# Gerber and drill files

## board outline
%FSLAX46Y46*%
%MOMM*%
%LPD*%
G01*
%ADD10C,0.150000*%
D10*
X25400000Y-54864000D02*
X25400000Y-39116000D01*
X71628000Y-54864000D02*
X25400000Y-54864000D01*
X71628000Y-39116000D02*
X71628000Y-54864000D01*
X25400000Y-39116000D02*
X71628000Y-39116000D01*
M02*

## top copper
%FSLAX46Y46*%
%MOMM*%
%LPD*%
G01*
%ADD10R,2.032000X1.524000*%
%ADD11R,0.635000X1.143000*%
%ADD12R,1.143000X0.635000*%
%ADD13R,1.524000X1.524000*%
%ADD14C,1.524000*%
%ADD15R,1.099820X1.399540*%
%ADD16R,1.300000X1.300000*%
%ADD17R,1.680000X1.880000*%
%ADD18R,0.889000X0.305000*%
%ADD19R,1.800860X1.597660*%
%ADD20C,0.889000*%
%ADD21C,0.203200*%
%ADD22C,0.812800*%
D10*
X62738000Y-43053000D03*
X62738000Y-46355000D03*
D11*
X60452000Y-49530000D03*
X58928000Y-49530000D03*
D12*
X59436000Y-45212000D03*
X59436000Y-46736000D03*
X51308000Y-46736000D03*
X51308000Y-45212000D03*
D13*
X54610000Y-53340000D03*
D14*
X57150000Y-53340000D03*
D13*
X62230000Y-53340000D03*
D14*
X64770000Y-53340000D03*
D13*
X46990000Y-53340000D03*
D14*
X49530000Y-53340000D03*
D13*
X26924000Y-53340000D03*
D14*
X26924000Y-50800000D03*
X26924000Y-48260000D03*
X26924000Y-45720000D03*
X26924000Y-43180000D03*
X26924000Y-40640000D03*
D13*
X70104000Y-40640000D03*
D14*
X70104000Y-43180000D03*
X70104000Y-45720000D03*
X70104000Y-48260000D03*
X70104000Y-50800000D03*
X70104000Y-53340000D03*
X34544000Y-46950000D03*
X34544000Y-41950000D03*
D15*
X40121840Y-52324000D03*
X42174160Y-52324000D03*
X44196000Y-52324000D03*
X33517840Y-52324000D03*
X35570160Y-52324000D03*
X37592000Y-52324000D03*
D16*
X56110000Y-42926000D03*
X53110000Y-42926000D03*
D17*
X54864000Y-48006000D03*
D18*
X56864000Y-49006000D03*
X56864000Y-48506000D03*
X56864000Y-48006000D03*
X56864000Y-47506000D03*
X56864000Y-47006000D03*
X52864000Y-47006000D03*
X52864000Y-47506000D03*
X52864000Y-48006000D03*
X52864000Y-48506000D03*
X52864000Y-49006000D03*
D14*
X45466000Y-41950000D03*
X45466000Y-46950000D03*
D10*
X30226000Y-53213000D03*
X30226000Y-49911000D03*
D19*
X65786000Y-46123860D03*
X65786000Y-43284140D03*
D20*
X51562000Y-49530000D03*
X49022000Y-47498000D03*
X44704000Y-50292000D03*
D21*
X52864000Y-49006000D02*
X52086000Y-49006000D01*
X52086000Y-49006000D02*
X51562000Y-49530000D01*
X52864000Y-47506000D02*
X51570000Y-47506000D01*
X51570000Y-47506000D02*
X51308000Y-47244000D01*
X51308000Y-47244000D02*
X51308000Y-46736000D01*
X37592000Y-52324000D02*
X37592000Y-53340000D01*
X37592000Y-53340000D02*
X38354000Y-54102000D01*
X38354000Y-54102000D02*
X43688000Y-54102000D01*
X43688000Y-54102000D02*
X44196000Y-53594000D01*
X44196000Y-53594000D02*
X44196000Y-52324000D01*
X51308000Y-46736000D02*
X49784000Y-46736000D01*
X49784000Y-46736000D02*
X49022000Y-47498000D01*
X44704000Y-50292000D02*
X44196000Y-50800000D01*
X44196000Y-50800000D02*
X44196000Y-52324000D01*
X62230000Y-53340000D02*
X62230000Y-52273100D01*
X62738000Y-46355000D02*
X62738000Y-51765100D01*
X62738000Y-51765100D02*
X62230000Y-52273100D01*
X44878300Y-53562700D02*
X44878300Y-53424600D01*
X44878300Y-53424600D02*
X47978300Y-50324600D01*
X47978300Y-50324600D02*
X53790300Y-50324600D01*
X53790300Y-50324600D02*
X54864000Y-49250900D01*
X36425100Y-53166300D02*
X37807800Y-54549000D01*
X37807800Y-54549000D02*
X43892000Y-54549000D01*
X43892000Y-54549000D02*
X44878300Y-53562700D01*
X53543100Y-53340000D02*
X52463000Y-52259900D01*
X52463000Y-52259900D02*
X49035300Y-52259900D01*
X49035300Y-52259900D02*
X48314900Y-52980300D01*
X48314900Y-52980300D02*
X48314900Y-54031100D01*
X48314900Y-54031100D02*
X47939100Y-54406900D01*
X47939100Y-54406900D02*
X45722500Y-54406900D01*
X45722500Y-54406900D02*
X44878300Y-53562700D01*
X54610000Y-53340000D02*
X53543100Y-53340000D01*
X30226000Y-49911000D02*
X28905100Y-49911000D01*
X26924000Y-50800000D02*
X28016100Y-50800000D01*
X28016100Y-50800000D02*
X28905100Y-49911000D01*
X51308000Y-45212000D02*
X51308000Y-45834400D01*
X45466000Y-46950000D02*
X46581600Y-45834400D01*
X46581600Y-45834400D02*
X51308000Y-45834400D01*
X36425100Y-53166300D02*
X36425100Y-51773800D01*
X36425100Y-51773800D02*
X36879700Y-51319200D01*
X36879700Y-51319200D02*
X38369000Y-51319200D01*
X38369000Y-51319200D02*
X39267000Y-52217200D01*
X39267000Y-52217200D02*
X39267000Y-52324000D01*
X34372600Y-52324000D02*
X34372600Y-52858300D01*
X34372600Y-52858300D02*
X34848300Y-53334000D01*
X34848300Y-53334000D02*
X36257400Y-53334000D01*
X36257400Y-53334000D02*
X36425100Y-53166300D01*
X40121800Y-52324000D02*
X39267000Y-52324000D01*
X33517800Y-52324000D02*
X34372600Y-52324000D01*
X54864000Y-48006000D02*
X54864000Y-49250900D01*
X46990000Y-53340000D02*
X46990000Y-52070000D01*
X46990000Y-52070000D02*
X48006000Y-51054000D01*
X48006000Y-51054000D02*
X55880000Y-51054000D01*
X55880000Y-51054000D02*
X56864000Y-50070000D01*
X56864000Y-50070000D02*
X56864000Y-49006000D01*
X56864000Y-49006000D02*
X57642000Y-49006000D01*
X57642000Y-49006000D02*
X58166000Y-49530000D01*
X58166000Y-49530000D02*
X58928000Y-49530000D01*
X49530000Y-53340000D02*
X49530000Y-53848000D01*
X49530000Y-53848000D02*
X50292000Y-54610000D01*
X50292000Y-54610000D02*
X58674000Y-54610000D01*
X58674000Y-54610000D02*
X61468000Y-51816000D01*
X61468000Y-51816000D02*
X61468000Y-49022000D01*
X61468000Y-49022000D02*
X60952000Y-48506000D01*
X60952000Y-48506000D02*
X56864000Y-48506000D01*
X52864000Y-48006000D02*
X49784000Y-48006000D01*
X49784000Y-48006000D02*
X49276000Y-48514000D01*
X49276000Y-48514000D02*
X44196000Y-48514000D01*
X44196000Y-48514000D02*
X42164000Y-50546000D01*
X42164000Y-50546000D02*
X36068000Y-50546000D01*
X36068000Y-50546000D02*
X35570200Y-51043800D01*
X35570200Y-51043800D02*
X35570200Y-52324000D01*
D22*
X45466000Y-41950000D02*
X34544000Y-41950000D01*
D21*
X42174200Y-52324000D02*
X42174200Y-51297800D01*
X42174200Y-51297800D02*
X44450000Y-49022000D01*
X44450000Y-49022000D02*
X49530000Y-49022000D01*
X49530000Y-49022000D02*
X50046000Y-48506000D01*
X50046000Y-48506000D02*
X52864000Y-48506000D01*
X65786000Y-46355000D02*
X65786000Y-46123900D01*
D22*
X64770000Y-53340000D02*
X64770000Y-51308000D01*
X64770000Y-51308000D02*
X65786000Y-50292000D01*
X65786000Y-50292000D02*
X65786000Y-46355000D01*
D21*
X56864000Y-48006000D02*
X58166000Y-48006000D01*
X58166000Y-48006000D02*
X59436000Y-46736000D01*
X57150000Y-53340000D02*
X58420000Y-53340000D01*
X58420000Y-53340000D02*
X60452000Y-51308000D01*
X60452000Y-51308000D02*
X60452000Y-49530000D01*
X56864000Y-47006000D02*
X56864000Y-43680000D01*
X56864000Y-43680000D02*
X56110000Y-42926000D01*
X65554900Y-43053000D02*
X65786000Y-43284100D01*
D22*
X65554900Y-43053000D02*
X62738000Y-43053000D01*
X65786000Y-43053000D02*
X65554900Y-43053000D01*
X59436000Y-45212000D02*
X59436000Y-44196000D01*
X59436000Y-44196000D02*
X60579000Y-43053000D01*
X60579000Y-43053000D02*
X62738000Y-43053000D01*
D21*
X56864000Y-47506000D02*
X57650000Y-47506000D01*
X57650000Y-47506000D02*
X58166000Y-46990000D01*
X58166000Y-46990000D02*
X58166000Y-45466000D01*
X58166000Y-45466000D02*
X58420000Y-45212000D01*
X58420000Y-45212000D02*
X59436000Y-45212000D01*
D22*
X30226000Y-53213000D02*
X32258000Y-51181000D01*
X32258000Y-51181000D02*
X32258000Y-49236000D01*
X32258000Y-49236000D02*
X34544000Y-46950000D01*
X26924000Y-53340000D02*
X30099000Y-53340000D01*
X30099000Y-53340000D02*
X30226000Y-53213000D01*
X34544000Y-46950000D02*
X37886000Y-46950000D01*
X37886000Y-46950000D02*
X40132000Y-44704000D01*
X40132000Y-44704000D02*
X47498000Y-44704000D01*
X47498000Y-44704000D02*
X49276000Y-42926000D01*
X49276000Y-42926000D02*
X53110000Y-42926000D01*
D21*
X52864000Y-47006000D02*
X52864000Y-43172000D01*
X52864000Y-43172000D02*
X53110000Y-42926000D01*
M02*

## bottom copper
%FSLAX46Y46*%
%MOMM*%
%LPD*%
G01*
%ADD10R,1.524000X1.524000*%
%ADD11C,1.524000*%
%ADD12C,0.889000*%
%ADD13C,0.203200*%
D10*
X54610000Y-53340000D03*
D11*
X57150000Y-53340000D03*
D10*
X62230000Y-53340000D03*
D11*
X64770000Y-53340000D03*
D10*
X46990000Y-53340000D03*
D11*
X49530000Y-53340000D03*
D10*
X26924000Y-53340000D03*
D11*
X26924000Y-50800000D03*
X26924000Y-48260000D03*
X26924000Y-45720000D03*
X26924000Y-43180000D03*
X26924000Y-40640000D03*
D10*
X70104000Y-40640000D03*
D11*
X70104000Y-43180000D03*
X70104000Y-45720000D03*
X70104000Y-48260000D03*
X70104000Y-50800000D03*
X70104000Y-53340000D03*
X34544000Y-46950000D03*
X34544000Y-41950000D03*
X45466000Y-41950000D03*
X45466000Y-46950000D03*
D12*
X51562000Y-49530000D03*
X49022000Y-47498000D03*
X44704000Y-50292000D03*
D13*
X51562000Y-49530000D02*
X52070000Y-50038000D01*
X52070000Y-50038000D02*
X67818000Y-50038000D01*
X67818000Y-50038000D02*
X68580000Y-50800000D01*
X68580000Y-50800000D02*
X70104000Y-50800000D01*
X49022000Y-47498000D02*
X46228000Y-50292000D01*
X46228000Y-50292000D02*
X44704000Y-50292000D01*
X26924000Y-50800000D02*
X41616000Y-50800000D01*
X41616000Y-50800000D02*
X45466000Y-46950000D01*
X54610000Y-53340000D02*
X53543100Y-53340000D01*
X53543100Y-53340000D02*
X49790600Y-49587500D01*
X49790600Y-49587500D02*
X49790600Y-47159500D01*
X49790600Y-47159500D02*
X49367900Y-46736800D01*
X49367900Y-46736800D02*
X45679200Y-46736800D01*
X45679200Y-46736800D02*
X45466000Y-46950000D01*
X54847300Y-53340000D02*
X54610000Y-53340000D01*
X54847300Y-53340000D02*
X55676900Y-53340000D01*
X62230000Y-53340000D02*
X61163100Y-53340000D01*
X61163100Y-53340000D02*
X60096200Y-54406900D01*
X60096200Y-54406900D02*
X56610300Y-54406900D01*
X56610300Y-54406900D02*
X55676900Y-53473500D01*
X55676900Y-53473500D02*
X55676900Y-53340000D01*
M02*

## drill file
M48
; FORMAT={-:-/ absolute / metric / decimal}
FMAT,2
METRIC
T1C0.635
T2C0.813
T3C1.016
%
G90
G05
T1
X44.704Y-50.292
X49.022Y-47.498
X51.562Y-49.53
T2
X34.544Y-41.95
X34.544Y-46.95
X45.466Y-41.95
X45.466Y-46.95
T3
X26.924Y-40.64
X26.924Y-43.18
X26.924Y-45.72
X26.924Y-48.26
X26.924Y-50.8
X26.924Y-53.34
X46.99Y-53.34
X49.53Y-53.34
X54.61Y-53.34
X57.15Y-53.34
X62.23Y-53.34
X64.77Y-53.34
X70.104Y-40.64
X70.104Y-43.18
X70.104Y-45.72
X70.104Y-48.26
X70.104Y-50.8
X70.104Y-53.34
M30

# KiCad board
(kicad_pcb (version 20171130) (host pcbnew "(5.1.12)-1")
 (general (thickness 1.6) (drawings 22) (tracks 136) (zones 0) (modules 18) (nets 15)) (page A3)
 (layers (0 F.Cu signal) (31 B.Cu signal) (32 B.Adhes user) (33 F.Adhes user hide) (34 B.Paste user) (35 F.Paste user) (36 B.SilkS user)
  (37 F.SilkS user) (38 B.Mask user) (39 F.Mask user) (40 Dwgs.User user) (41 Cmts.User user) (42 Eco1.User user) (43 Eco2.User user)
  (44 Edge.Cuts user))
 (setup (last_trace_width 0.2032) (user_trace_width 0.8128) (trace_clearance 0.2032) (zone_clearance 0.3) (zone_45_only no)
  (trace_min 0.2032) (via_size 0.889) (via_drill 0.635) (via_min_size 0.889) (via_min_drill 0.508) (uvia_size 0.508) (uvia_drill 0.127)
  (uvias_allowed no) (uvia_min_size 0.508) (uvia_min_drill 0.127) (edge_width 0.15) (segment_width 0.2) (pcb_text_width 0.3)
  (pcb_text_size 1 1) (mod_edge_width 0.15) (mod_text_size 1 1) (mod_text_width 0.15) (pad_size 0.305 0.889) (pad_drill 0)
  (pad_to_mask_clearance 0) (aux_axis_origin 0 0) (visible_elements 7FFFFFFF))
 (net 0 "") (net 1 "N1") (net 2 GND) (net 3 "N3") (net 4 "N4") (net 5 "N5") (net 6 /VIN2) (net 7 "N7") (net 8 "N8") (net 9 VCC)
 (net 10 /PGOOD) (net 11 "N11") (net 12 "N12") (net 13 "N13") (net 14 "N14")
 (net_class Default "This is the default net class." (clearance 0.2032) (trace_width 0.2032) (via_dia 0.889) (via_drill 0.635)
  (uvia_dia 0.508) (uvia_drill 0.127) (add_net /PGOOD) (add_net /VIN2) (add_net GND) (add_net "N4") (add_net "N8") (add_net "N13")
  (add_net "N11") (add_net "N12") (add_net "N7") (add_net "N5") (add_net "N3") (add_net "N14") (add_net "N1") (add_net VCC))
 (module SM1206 (layer F.Cu) (at 62.738 44.704 270)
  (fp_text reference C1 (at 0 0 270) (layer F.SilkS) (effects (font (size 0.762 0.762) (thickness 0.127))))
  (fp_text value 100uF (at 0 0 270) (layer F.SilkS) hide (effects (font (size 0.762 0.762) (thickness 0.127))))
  (pad 1 smd rect (at -1.651 0 270) (size 1.524 2.032) (layers F.Cu F.Paste F.Mask) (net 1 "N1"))
  (pad 2 smd rect (at 1.651 0 270) (size 1.524 2.032) (layers F.Cu F.Paste F.Mask) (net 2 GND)))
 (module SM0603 (layer F.Cu) (at 59.69 49.53 180)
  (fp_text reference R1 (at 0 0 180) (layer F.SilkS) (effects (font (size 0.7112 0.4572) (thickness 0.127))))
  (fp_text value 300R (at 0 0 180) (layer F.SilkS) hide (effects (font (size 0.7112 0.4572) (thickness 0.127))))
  (pad 1 smd rect (at -0.762 0 180) (size 0.635 1.143) (layers F.Cu F.Paste F.Mask) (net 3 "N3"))
  (pad 2 smd rect (at 0.762 0 180) (size 0.635 1.143) (layers F.Cu F.Paste F.Mask) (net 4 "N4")))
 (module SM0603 (layer F.Cu) (at 59.436 45.974 270)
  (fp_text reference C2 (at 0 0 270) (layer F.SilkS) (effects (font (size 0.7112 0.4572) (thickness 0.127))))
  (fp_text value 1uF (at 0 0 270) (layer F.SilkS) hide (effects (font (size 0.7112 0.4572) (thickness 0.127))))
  (pad 1 smd rect (at -0.762 0 270) (size 0.635 1.143) (layers F.Cu F.Paste F.Mask) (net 1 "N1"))
  (pad 2 smd rect (at 0.762 0 270) (size 0.635 1.143) (layers F.Cu F.Paste F.Mask) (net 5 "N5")))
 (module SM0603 (layer F.Cu) (at 51.308 45.974 90)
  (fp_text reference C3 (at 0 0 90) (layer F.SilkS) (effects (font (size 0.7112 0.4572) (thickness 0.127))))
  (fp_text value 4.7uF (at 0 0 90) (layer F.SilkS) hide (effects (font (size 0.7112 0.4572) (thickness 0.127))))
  (pad 1 smd rect (at -0.762 0 90) (size 0.635 1.143) (layers F.Cu F.Paste F.Mask) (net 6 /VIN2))
  (pad 2 smd rect (at 0.762 0 90) (size 0.635 1.143) (layers F.Cu F.Paste F.Mask) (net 2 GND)))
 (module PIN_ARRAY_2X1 (layer F.Cu) (at 55.88 53.34)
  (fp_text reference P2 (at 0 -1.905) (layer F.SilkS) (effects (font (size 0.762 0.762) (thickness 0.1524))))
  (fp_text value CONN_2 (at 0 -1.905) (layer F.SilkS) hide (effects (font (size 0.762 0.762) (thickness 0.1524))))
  (pad 1 thru_hole rect (at -1.27 0) (size 1.524 1.524) (drill 1.016) (layers *.Cu *.Mask F.SilkS) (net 2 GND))
  (pad 2 thru_hole circle (at 1.27 0) (size 1.524 1.524) (drill 1.016) (layers *.Cu *.Mask F.SilkS) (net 3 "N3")))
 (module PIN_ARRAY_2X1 (layer F.Cu) (at 63.5 53.34)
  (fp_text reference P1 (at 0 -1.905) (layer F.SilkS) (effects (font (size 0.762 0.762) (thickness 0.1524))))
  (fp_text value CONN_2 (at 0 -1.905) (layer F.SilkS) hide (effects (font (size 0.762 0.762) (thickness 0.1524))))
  (pad 1 thru_hole rect (at -1.27 0) (size 1.524 1.524) (drill 1.016) (layers *.Cu *.Mask F.SilkS) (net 2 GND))
  (pad 2 thru_hole circle (at 1.27 0) (size 1.524 1.524) (drill 1.016) (layers *.Cu *.Mask F.SilkS) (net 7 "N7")))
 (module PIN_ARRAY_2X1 (layer F.Cu) (at 48.26 53.34)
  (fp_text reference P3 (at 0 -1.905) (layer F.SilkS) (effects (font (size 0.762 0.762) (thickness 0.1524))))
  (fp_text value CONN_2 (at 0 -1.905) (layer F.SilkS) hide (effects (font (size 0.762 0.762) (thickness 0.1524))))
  (pad 1 thru_hole rect (at -1.27 0) (size 1.524 1.524) (drill 1.016) (layers *.Cu *.Mask F.SilkS) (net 4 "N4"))
  (pad 2 thru_hole circle (at 1.27 0) (size 1.524 1.524) (drill 1.016) (layers *.Cu *.Mask F.SilkS) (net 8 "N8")))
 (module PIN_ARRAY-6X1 (layer F.Cu) (at 26.924 46.99 90)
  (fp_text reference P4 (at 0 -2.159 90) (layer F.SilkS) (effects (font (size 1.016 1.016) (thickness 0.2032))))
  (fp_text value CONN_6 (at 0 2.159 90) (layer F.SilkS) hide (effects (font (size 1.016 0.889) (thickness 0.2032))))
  (pad 1 thru_hole rect (at -6.35 0 90) (size 1.524 1.524) (drill 1.016) (layers *.Cu *.Mask F.SilkS) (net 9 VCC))
  (pad 2 thru_hole circle (at -3.81 0 90) (size 1.524 1.524) (drill 1.016) (layers *.Cu *.Mask F.SilkS) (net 2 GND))
  (pad 3 thru_hole circle (at -1.27 0 90) (size 1.524 1.524) (drill 1.016) (layers *.Cu *.Mask F.SilkS))
  (pad 4 thru_hole circle (at 1.27 0 90) (size 1.524 1.524) (drill 1.016) (layers *.Cu *.Mask F.SilkS))
  (pad 5 thru_hole circle (at 3.81 0 90) (size 1.524 1.524) (drill 1.016) (layers *.Cu *.Mask F.SilkS))
  (pad 6 thru_hole circle (at 6.35 0 90) (size 1.524 1.524) (drill 1.016) (layers *.Cu *.Mask F.SilkS)))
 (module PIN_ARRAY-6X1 (layer F.Cu) (at 70.104 46.99 270)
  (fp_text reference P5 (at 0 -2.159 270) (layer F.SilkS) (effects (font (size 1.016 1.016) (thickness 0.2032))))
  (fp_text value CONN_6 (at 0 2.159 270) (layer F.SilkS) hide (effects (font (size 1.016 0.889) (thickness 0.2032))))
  (pad 1 thru_hole rect (at -6.35 0 270) (size 1.524 1.524) (drill 1.016) (layers *.Cu *.Mask F.SilkS))
  (pad 2 thru_hole circle (at -3.81 0 270) (size 1.524 1.524) (drill 1.016) (layers *.Cu *.Mask F.SilkS))
  (pad 3 thru_hole circle (at -1.27 0 270) (size 1.524 1.524) (drill 1.016) (layers *.Cu *.Mask F.SilkS))
  (pad 4 thru_hole circle (at 1.27 0 270) (size 1.524 1.524) (drill 1.016) (layers *.Cu *.Mask F.SilkS))
  (pad 5 thru_hole circle (at 3.81 0 270) (size 1.524 1.524) (drill 1.016) (layers *.Cu *.Mask F.SilkS) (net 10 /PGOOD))
  (pad 6 thru_hole circle (at 6.35 0 270) (size 1.524 1.524) (drill 1.016) (layers *.Cu *.Mask F.SilkS)))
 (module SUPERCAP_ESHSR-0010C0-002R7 (layer F.Cu) (at 34.544 44.45 90)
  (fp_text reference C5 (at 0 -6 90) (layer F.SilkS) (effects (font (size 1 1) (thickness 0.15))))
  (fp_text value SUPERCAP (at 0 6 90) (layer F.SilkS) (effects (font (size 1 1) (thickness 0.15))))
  (pad 1 thru_hole circle (at -2.5 0 90) (size 1.524 1.524) (drill 0.8128) (layers *.Cu *.Mask F.SilkS) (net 9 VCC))
  (pad 2 thru_hole circle (at 2.5 0 90) (size 1.524 1.524) (drill 0.8128) (layers *.Cu *.Mask F.SilkS) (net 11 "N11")))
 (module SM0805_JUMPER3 (layer F.Cu) (at 42.164 52.324)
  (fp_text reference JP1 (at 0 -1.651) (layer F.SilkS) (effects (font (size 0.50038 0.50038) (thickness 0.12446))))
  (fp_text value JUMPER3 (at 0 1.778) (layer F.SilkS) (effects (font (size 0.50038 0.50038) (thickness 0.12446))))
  (pad 1 smd rect (at -2.04216 0) (size 1.09982 1.39954) (layers F.Cu F.Paste F.Mask) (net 2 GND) (solder_mask_margin 0.09906))
  (pad 2 smd rect (at 0.01016 0) (size 1.09982 1.39954) (layers F.Cu F.Paste F.Mask) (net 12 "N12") (solder_mask_margin 0.09906))
  (pad 3 smd rect (at 2.032 0) (size 1.09982 1.39954) (layers F.Cu F.Paste F.Mask) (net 6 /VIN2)))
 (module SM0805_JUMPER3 (layer F.Cu) (at 35.56 52.324)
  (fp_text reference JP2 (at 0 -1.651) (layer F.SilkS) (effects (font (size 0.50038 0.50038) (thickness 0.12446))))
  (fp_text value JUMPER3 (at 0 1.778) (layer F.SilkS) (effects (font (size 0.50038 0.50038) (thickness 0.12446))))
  (pad 1 smd rect (at -2.04216 0) (size 1.09982 1.39954) (layers F.Cu F.Paste F.Mask) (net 2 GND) (solder_mask_margin 0.09906))
  (pad 2 smd rect (at 0.01016 0) (size 1.09982 1.39954) (layers F.Cu F.Paste F.Mask) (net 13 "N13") (solder_mask_margin 0.09906))
  (pad 3 smd rect (at 2.032 0) (size 1.09982 1.39954) (layers F.Cu F.Paste F.Mask) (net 6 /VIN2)))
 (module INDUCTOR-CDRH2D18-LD (layer F.Cu) (at 54.61 42.926 180)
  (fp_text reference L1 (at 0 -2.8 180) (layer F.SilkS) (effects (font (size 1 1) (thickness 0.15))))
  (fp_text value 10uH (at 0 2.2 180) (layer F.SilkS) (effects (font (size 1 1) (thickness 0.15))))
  (pad 1 smd rect (at -1.5 0 180) (size 1.3 1.3) (layers F.Cu F.Paste F.Mask) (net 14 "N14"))
  (pad 2 smd rect (at 1.5 0 180) (size 1.3 1.3) (layers F.Cu F.Paste F.Mask) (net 9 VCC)))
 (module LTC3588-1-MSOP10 (layer F.Cu) (at 54.864 48.006 90) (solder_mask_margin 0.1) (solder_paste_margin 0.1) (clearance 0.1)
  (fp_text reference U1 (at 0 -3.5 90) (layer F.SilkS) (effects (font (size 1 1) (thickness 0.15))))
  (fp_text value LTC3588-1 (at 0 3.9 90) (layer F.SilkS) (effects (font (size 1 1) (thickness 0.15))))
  (pad 11 smd rect (at 0 0 90) (size 1.88 1.68) (layers F.Cu F.Paste F.Mask) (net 2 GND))
  (pad 1 smd rect (at -1 2 90) (size 0.305 0.889) (layers F.Cu F.Paste F.Mask) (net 4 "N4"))
  (pad 2 smd rect (at -0.5 2 90) (size 0.305 0.889) (layers F.Cu F.Paste F.Mask) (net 8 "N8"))
  (pad 3 smd rect (at 0 2 90) (size 0.305 0.889) (layers F.Cu F.Paste F.Mask) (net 5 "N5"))
  (pad 4 smd rect (at 0.5 2 90) (size 0.305 0.889) (layers F.Cu F.Paste F.Mask) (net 1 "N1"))
  (pad 5 smd rect (at 1 2 90) (size 0.305 0.889) (layers F.Cu F.Paste F.Mask) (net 14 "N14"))
  (pad 6 smd rect (at 1 -2 90) (size 0.305 0.889) (layers F.Cu F.Paste F.Mask) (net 9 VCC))
  (pad 7 smd rect (at 0.5 -2 90) (size 0.305 0.889) (layers F.Cu F.Paste F.Mask) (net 6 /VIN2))
  (pad 8 smd rect (at 0 -2 90) (size 0.305 0.889) (layers F.Cu F.Paste F.Mask) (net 13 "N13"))
  (pad 9 smd rect (at -0.5 -2 90) (size 0.305 0.889) (layers F.Cu F.Paste F.Mask) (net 12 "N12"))
  (pad 10 smd rect (at -1 -2 90) (size 0.305 0.889) (layers F.Cu F.Paste F.Mask) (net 10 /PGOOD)))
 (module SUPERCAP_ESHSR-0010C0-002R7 (layer F.Cu) (at 45.466 44.45 270)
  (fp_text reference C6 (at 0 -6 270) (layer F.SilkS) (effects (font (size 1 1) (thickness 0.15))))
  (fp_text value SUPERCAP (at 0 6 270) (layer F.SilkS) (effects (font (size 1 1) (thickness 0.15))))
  (pad 1 thru_hole circle (at -2.5 0 270) (size 1.524 1.524) (drill 0.8128) (layers *.Cu *.Mask F.SilkS) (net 11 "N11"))
  (pad 2 thru_hole circle (at 2.5 0 270) (size 1.524 1.524) (drill 0.8128) (layers *.Cu *.Mask F.SilkS) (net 2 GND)))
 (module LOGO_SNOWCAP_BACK (layer B.Cu) (at 59.436 44.45)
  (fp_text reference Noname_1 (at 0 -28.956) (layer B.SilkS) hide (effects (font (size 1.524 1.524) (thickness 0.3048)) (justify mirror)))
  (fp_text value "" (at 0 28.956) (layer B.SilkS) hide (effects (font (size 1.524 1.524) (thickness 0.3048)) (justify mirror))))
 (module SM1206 (layer F.Cu) (at 30.226 51.562 90)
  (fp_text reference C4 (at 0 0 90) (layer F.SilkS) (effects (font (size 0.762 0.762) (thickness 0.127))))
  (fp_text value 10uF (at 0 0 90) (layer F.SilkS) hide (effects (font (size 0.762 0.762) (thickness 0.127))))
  (pad 1 smd rect (at -1.651 0 90) (size 1.524 2.032) (layers F.Cu F.Paste F.Mask) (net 9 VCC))
  (pad 2 smd rect (at 1.651 0 90) (size 1.524 2.032) (layers F.Cu F.Paste F.Mask) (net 2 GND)))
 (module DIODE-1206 (layer F.Cu) (at 65.786 44.704 90)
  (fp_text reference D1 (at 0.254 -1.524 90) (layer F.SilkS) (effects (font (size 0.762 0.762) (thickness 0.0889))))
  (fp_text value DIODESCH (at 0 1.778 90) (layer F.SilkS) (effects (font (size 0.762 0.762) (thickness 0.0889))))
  (pad 1 smd rect (at -1.41986 0 90) (size 1.59766 1.80086) (layers F.Cu F.Paste F.Mask) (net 7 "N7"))
  (pad 2 smd rect (at 1.41986 0 90) (size 1.59766 1.80086) (layers F.Cu F.Paste F.Mask) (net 1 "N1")))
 (gr_line (start 25.4 54.864) (end 25.4 39.116) (angle 90) (layer Edge.Cuts) (width 0.15))
 (gr_line (start 71.628 54.864) (end 25.4 54.864) (angle 90) (layer Edge.Cuts) (width 0.15))
 (gr_line (start 71.628 39.116) (end 71.628 54.864) (angle 90) (layer Edge.Cuts) (width 0.15))
 (gr_line (start 25.4 39.116) (end 71.628 39.116) (angle 90) (layer Edge.Cuts) (width 0.15))
 (segment (start 52.864 49.006) (end 52.086 49.006) (width 0.2032) (layer F.Cu) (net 10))
 (segment (start 52.086 49.006) (end 51.562 49.53) (width 0.2032) (layer F.Cu) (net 10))
 (segment (start 51.562 49.53) (end 52.07 50.038) (width 0.2032) (layer B.Cu) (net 10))
 (segment (start 52.07 50.038) (end 67.818 50.038) (width 0.2032) (layer B.Cu) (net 10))
 (segment (start 67.818 50.038) (end 68.58 50.8) (width 0.2032) (layer B.Cu) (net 10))
 (segment (start 68.58 50.8) (end 70.104 50.8) (width 0.2032) (layer B.Cu) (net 10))
 (via (at 51.562 49.53) (size 0.889) (layers F.Cu B.Cu) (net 10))
 (segment (start 52.864 47.506) (end 51.57 47.506) (width 0.2032) (layer F.Cu) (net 6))
 (segment (start 51.57 47.506) (end 51.308 47.244) (width 0.2032) (layer F.Cu) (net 6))
 (segment (start 51.308 47.244) (end 51.308 46.736) (width 0.2032) (layer F.Cu) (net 6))
 (segment (start 37.592 52.324) (end 37.592 53.34) (width 0.2032) (layer F.Cu) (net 6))
 (segment (start 37.592 53.34) (end 38.354 54.102) (width 0.2032) (layer F.Cu) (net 6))
 (segment (start 38.354 54.102) (end 43.688 54.102) (width 0.2032) (layer F.Cu) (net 6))
 (segment (start 43.688 54.102) (end 44.196 53.594) (width 0.2032) (layer F.Cu) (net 6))
 (segment (start 44.196 53.594) (end 44.196 52.324) (width 0.2032) (layer F.Cu) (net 6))
 (segment (start 51.308 46.736) (end 49.784 46.736) (width 0.2032) (layer F.Cu) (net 6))
 (segment (start 49.784 46.736) (end 49.022 47.498) (width 0.2032) (layer F.Cu) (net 6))
 (segment (start 49.022 47.498) (end 46.228 50.292) (width 0.2032) (layer B.Cu) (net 6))
 (segment (start 46.228 50.292) (end 44.704 50.292) (width 0.2032) (layer B.Cu) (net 6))
 (segment (start 44.704 50.292) (end 44.196 50.8) (width 0.2032) (layer F.Cu) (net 6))
 (segment (start 44.196 50.8) (end 44.196 52.324) (width 0.2032) (layer F.Cu) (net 6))
 (via (at 49.022 47.498) (size 0.889) (layers F.Cu B.Cu) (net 6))
 (via (at 44.704 50.292) (size 0.889) (layers F.Cu B.Cu) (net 6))
 (segment (start 62.23 53.34) (end 62.23 52.2731) (width 0.2032) (layer F.Cu) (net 2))
 (segment (start 62.738 46.355) (end 62.738 51.7651) (width 0.2032) (layer F.Cu) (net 2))
 (segment (start 62.738 51.7651) (end 62.23 52.2731) (width 0.2032) (layer F.Cu) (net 2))
 (segment (start 26.924 50.8) (end 41.616 50.8) (width 0.2032) (layer B.Cu) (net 2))
 (segment (start 41.616 50.8) (end 45.466 46.95) (width 0.2032) (layer B.Cu) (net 2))
 (segment (start 44.8783 53.5627) (end 44.8783 53.4246) (width 0.2032) (layer F.Cu) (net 2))
 (segment (start 44.8783 53.4246) (end 47.9783 50.3246) (width 0.2032) (layer F.Cu) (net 2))
 (segment (start 47.9783 50.3246) (end 53.7903 50.3246) (width 0.2032) (layer F.Cu) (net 2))
 (segment (start 53.7903 50.3246) (end 54.864 49.2509) (width 0.2032) (layer F.Cu) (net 2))
 (segment (start 36.4251 53.1663) (end 37.8078 54.549) (width 0.2032) (layer F.Cu) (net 2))
 (segment (start 37.8078 54.549) (end 43.892 54.549) (width 0.2032) (layer F.Cu) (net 2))
 (segment (start 43.892 54.549) (end 44.8783 53.5627) (width 0.2032) (layer F.Cu) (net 2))
 (segment (start 53.5431 53.34) (end 52.463 52.2599) (width 0.2032) (layer F.Cu) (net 2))
 (segment (start 52.463 52.2599) (end 49.0353 52.2599) (width 0.2032) (layer F.Cu) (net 2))
 (segment (start 49.0353 52.2599) (end 48.3149 52.9803) (width 0.2032) (layer F.Cu) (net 2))
 (segment (start 48.3149 52.9803) (end 48.3149 54.0311) (width 0.2032) (layer F.Cu) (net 2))
 (segment (start 48.3149 54.0311) (end 47.9391 54.4069) (width 0.2032) (layer F.Cu) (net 2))
 (segment (start 47.9391 54.4069) (end 45.7225 54.4069) (width 0.2032) (layer F.Cu) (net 2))
 (segment (start 45.7225 54.4069) (end 44.8783 53.5627) (width 0.2032) (layer F.Cu) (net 2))
 (segment (start 54.61 53.34) (end 53.5431 53.34) (width 0.2032) (layer F.Cu) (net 2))
 (segment (start 54.61 53.34) (end 53.5431 53.34) (width 0.2032) (layer B.Cu) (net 2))
 (segment (start 53.5431 53.34) (end 49.7906 49.5875) (width 0.2032) (layer B.Cu) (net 2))
 (segment (start 49.7906 49.5875) (end 49.7906 47.1595) (width 0.2032) (layer B.Cu) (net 2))
 (segment (start 49.7906 47.1595) (end 49.3679 46.7368) (width 0.2032) (layer B.Cu) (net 2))
 (segment (start 49.3679 46.7368) (end 45.6792 46.7368) (width 0.2032) (layer B.Cu) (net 2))
 (segment (start 45.6792 46.7368) (end 45.466 46.95) (width 0.2032) (layer B.Cu) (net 2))
 (segment (start 54.8473 53.34) (end 54.61 53.34) (width 0.2032) (layer B.Cu) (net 2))
 (segment (start 54.8473 53.34) (end 55.6769 53.34) (width 0.2032) (layer B.Cu) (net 2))
 (segment (start 62.23 53.34) (end 61.1631 53.34) (width 0.2032) (layer B.Cu) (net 2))
 (segment (start 61.1631 53.34) (end 60.0962 54.4069) (width 0.2032) (layer B.Cu) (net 2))
 (segment (start 60.0962 54.4069) (end 56.6103 54.4069) (width 0.2032) (layer B.Cu) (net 2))
 (segment (start 56.6103 54.4069) (end 55.6769 53.4735) (width 0.2032) (layer B.Cu) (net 2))
 (segment (start 55.6769 53.4735) (end 55.6769 53.34) (width 0.2032) (layer B.Cu) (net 2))
 (segment (start 30.226 49.911) (end 28.9051 49.911) (width 0.2032) (layer F.Cu) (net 2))
 (segment (start 26.924 50.8) (end 28.0161 50.8) (width 0.2032) (layer F.Cu) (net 2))
 (segment (start 28.0161 50.8) (end 28.9051 49.911) (width 0.2032) (layer F.Cu) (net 2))
 (segment (start 51.308 45.212) (end 51.308 45.8344) (width 0.2032) (layer F.Cu) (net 2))
 (segment (start 45.466 46.95) (end 46.5816 45.8344) (width 0.2032) (layer F.Cu) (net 2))
 (segment (start 46.5816 45.8344) (end 51.308 45.8344) (width 0.2032) (layer F.Cu) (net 2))
 (segment (start 36.4251 53.1663) (end 36.4251 51.7738) (width 0.2032) (layer F.Cu) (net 2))
 (segment (start 36.4251 51.7738) (end 36.8797 51.3192) (width 0.2032) (layer F.Cu) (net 2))
 (segment (start 36.8797 51.3192) (end 38.369 51.3192) (width 0.2032) (layer F.Cu) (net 2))
 (segment (start 38.369 51.3192) (end 39.267 52.2172) (width 0.2032) (layer F.Cu) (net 2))
 (segment (start 39.267 52.2172) (end 39.267 52.324) (width 0.2032) (layer F.Cu) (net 2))
 (segment (start 34.3726 52.324) (end 34.3726 52.8583) (width 0.2032) (layer F.Cu) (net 2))
 (segment (start 34.3726 52.8583) (end 34.8483 53.334) (width 0.2032) (layer F.Cu) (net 2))
 (segment (start 34.8483 53.334) (end 36.2574 53.334) (width 0.2032) (layer F.Cu) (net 2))
 (segment (start 36.2574 53.334) (end 36.4251 53.1663) (width 0.2032) (layer F.Cu) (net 2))
 (segment (start 40.1218 52.324) (end 39.267 52.324) (width 0.2032) (layer F.Cu) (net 2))
 (segment (start 33.5178 52.324) (end 34.3726 52.324) (width 0.2032) (layer F.Cu) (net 2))
 (segment (start 54.864 48.006) (end 54.864 49.2509) (width 0.2032) (layer F.Cu) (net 2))
 (segment (start 46.99 53.34) (end 46.99 52.07) (width 0.2032) (layer F.Cu) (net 4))
 (segment (start 46.99 52.07) (end 48.006 51.054) (width 0.2032) (layer F.Cu) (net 4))
 (segment (start 48.006 51.054) (end 55.88 51.054) (width 0.2032) (layer F.Cu) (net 4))
 (segment (start 55.88 51.054) (end 56.864 50.07) (width 0.2032) (layer F.Cu) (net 4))
 (segment (start 56.864 50.07) (end 56.864 49.006) (width 0.2032) (layer F.Cu) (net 4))
 (segment (start 56.864 49.006) (end 57.642 49.006) (width 0.2032) (layer F.Cu) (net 4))
 (segment (start 57.642 49.006) (end 58.166 49.53) (width 0.2032) (layer F.Cu) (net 4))
 (segment (start 58.166 49.53) (end 58.928 49.53) (width 0.2032) (layer F.Cu) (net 4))
 (segment (start 49.53 53.34) (end 49.53 53.848) (width 0.2032) (layer F.Cu) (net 8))
 (segment (start 49.53 53.848) (end 50.292 54.61) (width 0.2032) (layer F.Cu) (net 8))
 (segment (start 50.292 54.61) (end 58.674 54.61) (width 0.2032) (layer F.Cu) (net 8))
 (segment (start 58.674 54.61) (end 61.468 51.816) (width 0.2032) (layer F.Cu) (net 8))
 (segment (start 61.468 51.816) (end 61.468 49.022) (width 0.2032) (layer F.Cu) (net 8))
 (segment (start 61.468 49.022) (end 60.952 48.506) (width 0.2032) (layer F.Cu) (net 8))
 (segment (start 60.952 48.506) (end 56.864 48.506) (width 0.2032) (layer F.Cu) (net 8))
 (segment (start 52.864 48.006) (end 49.784 48.006) (width 0.2032) (layer F.Cu) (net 13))
 (segment (start 49.784 48.006) (end 49.276 48.514) (width 0.2032) (layer F.Cu) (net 13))
 (segment (start 49.276 48.514) (end 44.196 48.514) (width 0.2032) (layer F.Cu) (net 13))
 (segment (start 44.196 48.514) (end 42.164 50.546) (width 0.2032) (layer F.Cu) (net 13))
 (segment (start 42.164 50.546) (end 36.068 50.546) (width 0.2032) (layer F.Cu) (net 13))
 (segment (start 36.068 50.546) (end 35.5702 51.0438) (width 0.2032) (layer F.Cu) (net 13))
 (segment (start 35.5702 51.0438) (end 35.5702 52.324) (width 0.2032) (layer F.Cu) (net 13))
 (segment (start 45.466 41.95) (end 34.544 41.95) (width 0.8128) (layer F.Cu) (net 11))
 (segment (start 42.1742 52.324) (end 42.1742 51.2978) (width 0.2032) (layer F.Cu) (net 12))
 (segment (start 42.1742 51.2978) (end 44.45 49.022) (width 0.2032) (layer F.Cu) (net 12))
 (segment (start 44.45 49.022) (end 49.53 49.022) (width 0.2032) (layer F.Cu) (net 12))
 (segment (start 49.53 49.022) (end 50.046 48.506) (width 0.2032) (layer F.Cu) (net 12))
 (segment (start 50.046 48.506) (end 52.864 48.506) (width 0.2032) (layer F.Cu) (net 12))
 (segment (start 65.786 46.355) (end 65.786 46.1239) (width 0.2032) (layer F.Cu) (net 7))
 (segment (start 64.77 53.34) (end 64.77 51.308) (width 0.8128) (layer F.Cu) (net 7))
 (segment (start 64.77 51.308) (end 65.786 50.292) (width 0.8128) (layer F.Cu) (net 7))
 (segment (start 65.786 50.292) (end 65.786 46.355) (width 0.8128) (layer F.Cu) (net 7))
 (segment (start 56.864 48.006) (end 58.166 48.006) (width 0.2032) (layer F.Cu) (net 5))
 (segment (start 58.166 48.006) (end 59.436 46.736) (width 0.2032) (layer F.Cu) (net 5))
 (segment (start 57.15 53.34) (end 58.42 53.34) (width 0.2032) (layer F.Cu) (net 3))
 (segment (start 58.42 53.34) (end 60.452 51.308) (width 0.2032) (layer F.Cu) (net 3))
 (segment (start 60.452 51.308) (end 60.452 49.53) (width 0.2032) (layer F.Cu) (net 3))
 (segment (start 56.864 47.006) (end 56.864 43.68) (width 0.2032) (layer F.Cu) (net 14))
 (segment (start 56.864 43.68) (end 56.11 42.926) (width 0.2032) (layer F.Cu) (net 14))
 (segment (start 65.5549 43.053) (end 65.786 43.2841) (width 0.2032) (layer F.Cu) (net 1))
 (segment (start 65.5549 43.053) (end 62.738 43.053) (width 0.8128) (layer F.Cu) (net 1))
 (segment (start 65.786 43.053) (end 65.5549 43.053) (width 0.8128) (layer F.Cu) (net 1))
 (segment (start 59.436 45.212) (end 59.436 44.196) (width 0.8128) (layer F.Cu) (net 1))
 (segment (start 59.436 44.196) (end 60.579 43.053) (width 0.8128) (layer F.Cu) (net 1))
 (segment (start 60.579 43.053) (end 62.738 43.053) (width 0.8128) (layer F.Cu) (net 1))
 (segment (start 56.864 47.506) (end 57.65 47.506) (width 0.2032) (layer F.Cu) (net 1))
 (segment (start 57.65 47.506) (end 58.166 46.99) (width 0.2032) (layer F.Cu) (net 1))
 (segment (start 58.166 46.99) (end 58.166 45.466) (width 0.2032) (layer F.Cu) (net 1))
 (segment (start 58.166 45.466) (end 58.42 45.212) (width 0.2032) (layer F.Cu) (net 1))
 (segment (start 58.42 45.212) (end 59.436 45.212) (width 0.2032) (layer F.Cu) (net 1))
 (segment (start 30.226 53.213) (end 32.258 51.181) (width 0.8128) (layer F.Cu) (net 9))
 (segment (start 32.258 51.181) (end 32.258 49.236) (width 0.8128) (layer F.Cu) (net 9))
 (segment (start 32.258 49.236) (end 34.544 46.95) (width 0.8128) (layer F.Cu) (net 9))
 (segment (start 26.924 53.34) (end 30.099 53.34) (width 0.8128) (layer F.Cu) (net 9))
 (segment (start 30.099 53.34) (end 30.226 53.213) (width 0.8128) (layer F.Cu) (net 9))
 (segment (start 34.544 46.95) (end 37.886 46.95) (width 0.8128) (layer F.Cu) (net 9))
 (segment (start 37.886 46.95) (end 40.132 44.704) (width 0.8128) (layer F.Cu) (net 9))
 (segment (start 40.132 44.704) (end 47.498 44.704) (width 0.8128) (layer F.Cu) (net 9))
 (segment (start 47.498 44.704) (end 49.276 42.926) (width 0.8128) (layer F.Cu) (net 9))
 (segment (start 49.276 42.926) (end 53.11 42.926) (width 0.8128) (layer F.Cu) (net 9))
 (segment (start 52.864 47.006) (end 52.864 43.172) (width 0.2032) (layer F.Cu) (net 9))
 (segment (start 52.864 43.172) (end 53.11 42.926) (width 0.2032) (layer F.Cu) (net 9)))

